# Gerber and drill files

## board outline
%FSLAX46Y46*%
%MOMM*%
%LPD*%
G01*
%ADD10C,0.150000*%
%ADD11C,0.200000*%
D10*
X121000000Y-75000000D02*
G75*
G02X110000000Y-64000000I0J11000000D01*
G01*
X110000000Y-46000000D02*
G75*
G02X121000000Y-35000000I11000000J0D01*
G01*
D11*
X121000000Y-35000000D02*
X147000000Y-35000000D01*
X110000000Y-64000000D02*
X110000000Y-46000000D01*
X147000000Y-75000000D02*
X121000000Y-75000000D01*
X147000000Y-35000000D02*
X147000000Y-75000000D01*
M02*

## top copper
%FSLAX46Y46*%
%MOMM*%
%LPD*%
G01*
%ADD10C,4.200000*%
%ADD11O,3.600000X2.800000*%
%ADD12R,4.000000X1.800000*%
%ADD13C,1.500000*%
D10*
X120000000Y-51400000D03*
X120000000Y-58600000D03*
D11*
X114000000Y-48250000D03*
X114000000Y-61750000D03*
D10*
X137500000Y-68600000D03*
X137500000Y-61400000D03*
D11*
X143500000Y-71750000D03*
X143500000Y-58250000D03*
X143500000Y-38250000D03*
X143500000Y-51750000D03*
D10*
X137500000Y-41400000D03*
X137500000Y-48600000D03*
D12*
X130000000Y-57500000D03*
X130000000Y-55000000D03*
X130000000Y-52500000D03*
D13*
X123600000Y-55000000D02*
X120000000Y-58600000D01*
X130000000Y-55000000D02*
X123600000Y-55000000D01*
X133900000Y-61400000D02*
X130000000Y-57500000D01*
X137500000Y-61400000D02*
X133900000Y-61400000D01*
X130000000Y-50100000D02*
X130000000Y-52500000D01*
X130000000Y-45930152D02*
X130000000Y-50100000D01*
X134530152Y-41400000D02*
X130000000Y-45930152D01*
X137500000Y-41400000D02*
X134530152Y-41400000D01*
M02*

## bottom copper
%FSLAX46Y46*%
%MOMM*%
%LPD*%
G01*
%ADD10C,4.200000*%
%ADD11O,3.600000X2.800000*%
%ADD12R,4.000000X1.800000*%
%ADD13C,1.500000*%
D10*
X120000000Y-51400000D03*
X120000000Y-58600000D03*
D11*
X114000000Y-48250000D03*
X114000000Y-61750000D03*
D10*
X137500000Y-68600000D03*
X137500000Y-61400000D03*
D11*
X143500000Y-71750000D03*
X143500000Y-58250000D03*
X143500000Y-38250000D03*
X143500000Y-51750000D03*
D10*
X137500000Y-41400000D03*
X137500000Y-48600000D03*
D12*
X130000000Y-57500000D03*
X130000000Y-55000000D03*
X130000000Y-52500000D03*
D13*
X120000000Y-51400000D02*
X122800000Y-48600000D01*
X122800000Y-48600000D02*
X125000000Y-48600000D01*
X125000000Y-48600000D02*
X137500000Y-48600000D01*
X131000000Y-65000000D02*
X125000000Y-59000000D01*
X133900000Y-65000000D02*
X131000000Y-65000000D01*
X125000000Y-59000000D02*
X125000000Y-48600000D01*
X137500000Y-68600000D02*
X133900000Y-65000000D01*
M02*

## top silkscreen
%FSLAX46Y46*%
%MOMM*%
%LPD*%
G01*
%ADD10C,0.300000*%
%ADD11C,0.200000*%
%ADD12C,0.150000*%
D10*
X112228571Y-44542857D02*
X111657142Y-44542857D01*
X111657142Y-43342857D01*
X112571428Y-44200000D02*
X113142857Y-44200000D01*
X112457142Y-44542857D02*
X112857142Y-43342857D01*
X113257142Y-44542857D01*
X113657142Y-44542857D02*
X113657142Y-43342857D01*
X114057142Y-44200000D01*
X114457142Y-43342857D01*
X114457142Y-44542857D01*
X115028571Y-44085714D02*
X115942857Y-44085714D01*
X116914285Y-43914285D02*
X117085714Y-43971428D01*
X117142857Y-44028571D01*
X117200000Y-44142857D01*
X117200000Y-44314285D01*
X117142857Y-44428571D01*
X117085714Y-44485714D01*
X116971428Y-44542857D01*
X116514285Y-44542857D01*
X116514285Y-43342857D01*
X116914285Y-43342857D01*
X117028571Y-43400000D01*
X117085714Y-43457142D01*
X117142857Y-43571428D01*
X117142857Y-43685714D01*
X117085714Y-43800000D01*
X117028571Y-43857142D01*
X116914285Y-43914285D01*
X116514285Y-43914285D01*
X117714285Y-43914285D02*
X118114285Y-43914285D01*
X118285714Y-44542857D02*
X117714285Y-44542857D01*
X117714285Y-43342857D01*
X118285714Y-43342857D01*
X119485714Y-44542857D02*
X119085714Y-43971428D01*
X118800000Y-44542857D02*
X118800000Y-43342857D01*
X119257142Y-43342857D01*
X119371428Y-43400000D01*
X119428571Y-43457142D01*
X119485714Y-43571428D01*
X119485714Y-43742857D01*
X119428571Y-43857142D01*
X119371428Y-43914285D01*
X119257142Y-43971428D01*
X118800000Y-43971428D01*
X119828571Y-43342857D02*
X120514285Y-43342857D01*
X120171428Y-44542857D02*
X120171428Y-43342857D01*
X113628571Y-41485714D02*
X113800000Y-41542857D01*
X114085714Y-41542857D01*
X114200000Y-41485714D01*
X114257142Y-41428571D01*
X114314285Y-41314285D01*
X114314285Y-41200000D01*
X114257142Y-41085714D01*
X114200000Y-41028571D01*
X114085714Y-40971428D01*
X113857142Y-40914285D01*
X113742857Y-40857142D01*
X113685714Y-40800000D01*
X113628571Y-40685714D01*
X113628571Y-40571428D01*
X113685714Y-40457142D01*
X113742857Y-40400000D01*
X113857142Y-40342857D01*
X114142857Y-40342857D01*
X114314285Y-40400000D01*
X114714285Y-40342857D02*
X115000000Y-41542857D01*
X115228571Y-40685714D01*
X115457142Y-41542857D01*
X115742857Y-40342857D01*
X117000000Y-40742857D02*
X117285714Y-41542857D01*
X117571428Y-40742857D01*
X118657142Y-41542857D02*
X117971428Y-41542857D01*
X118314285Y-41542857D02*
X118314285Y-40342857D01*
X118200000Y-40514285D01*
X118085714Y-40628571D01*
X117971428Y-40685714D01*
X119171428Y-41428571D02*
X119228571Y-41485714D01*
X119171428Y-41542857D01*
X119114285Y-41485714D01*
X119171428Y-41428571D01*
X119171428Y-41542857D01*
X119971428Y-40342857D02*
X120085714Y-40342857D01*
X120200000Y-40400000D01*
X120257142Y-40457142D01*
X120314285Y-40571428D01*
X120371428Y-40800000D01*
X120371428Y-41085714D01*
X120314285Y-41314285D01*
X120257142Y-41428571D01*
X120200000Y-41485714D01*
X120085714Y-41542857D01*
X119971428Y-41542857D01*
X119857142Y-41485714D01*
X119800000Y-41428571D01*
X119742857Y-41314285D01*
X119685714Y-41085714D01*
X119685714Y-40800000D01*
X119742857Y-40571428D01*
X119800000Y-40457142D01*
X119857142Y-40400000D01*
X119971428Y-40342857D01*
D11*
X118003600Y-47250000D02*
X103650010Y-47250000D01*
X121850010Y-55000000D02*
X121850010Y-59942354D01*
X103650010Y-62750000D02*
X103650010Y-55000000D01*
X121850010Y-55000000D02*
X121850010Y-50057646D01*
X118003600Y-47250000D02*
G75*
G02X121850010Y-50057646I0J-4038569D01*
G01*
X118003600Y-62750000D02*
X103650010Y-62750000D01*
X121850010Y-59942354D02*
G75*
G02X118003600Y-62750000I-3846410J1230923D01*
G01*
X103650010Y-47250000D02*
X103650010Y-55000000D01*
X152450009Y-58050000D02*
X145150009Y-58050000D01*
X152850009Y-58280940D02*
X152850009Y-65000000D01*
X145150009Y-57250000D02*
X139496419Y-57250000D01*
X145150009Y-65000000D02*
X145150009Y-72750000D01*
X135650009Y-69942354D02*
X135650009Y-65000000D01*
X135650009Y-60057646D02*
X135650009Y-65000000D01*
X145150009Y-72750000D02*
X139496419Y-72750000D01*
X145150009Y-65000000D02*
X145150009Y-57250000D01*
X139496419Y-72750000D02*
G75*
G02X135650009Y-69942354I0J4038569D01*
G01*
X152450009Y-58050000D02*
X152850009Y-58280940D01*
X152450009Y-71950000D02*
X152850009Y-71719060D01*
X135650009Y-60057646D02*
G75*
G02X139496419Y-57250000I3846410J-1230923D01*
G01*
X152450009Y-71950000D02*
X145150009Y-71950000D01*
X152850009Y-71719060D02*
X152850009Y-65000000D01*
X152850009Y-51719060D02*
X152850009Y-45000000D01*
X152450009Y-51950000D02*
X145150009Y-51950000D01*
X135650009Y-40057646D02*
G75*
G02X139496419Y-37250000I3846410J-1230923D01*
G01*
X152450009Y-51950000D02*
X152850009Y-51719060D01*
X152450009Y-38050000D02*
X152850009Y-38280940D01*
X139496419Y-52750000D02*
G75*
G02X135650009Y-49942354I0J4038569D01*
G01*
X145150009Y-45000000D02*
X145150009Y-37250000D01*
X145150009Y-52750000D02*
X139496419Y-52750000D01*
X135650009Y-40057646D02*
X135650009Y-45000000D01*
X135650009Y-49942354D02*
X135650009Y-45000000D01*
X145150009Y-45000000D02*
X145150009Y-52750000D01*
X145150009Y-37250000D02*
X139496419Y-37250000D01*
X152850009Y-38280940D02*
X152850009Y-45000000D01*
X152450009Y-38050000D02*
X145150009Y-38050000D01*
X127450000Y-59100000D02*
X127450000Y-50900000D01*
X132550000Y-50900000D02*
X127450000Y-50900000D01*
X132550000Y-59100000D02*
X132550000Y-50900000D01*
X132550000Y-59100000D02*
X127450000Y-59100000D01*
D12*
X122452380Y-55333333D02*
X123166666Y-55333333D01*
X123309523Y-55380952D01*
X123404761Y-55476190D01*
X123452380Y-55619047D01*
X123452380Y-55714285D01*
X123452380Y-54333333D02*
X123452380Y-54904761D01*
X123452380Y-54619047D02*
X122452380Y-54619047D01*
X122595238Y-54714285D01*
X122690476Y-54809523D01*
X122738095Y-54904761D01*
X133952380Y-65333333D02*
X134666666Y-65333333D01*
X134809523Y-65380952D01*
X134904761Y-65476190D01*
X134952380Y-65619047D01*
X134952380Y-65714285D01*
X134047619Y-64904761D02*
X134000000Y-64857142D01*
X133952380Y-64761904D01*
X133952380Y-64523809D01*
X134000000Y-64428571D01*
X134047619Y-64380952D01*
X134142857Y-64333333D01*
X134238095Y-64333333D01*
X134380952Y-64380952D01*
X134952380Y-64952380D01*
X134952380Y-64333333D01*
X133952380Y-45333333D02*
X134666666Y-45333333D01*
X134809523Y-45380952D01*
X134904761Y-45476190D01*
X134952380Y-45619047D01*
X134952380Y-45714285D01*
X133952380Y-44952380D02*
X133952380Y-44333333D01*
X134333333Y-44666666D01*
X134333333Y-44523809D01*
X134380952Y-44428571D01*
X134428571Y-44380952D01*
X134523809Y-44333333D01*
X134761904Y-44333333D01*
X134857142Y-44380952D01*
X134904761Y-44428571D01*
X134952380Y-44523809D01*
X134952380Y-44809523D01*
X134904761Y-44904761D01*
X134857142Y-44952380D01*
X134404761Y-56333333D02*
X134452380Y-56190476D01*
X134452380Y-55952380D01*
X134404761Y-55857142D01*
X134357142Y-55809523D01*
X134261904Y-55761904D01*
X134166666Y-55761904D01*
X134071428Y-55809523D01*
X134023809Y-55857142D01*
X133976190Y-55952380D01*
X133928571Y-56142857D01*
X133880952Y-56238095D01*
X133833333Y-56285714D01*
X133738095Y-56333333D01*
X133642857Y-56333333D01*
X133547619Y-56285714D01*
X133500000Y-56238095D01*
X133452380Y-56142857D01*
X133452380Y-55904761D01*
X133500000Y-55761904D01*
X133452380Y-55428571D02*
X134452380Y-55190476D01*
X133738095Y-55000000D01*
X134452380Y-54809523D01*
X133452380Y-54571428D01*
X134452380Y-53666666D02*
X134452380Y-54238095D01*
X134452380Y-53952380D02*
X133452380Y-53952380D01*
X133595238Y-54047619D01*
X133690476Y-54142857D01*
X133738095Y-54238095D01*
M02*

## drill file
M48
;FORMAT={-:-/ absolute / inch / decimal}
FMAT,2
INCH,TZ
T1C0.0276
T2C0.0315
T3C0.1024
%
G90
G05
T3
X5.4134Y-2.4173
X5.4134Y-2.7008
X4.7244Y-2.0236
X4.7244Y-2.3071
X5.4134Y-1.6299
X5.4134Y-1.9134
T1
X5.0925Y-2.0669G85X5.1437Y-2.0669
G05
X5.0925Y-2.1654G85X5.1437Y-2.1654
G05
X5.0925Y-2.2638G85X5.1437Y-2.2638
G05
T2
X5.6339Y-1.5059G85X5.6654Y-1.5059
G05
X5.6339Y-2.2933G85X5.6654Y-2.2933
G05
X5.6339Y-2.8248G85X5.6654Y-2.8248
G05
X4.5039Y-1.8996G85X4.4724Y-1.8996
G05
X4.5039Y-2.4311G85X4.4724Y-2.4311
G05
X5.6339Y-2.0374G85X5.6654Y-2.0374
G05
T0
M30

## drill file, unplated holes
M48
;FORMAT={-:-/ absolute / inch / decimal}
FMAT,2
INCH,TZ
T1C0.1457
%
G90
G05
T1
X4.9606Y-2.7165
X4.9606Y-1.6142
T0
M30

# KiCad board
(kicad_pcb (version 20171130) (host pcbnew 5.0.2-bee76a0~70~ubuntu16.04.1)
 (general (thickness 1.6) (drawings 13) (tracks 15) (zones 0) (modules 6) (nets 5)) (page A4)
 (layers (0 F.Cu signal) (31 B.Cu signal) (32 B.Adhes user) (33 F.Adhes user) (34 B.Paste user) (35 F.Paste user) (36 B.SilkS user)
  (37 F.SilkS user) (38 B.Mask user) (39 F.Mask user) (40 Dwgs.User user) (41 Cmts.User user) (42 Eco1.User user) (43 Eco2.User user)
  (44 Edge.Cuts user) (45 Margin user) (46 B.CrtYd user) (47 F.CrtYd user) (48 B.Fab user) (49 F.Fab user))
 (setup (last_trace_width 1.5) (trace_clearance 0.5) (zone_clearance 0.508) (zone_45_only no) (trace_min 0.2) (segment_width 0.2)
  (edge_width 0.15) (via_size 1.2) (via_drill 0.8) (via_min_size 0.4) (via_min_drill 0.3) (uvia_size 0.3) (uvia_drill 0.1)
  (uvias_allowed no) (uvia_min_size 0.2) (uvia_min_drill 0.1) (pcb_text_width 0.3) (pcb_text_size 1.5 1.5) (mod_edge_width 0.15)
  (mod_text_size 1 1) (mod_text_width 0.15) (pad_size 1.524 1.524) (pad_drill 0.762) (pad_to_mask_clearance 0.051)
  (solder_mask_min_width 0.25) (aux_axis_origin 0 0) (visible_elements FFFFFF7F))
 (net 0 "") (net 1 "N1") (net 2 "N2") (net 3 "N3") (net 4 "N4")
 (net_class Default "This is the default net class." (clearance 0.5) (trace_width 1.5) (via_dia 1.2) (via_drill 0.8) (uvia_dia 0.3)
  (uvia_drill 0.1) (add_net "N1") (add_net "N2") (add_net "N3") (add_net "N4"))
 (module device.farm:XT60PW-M (layer F.Cu) (at 120 55 270)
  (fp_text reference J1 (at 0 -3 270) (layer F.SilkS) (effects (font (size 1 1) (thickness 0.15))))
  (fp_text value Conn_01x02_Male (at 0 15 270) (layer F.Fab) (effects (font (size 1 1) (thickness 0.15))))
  (fp_line (start -7.75 1.9964) (end -7.75 16.34999) (layer F.SilkS) (width 0.2))
  (fp_line (start 0 -1.85001) (end 4.942354 -1.85001) (layer F.SilkS) (width 0.2))
  (fp_line (start 7.75 16.34999) (end 0 16.34999) (layer F.SilkS) (width 0.2))
  (fp_line (start 0 -1.85001) (end -4.942354 -1.85001) (layer F.SilkS) (width 0.2))
  (fp_arc (start -3.711431 1.9964) (end -4.942354 -1.85001) (angle -72.25435427) (layer F.SilkS) (width 0.2))
  (fp_line (start 7.75 1.9964) (end 7.75 16.34999) (layer F.SilkS) (width 0.2))
  (fp_arc (start 3.711431 1.9964) (end 7.75 1.9964) (angle -72.25435427) (layer F.SilkS) (width 0.2))
  (fp_line (start -7.75 16.34999) (end 0 16.34999) (layer F.SilkS) (width 0.2))
  (pad 1 thru_hole circle (at -3.6 0 270) (size 4.2 4.2) (drill 2.6) (layers *.Cu *.Mask) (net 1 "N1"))
  (pad 2 thru_hole circle (at 3.6 0 270) (size 4.2 4.2) (drill 2.6) (layers *.Cu *.Mask) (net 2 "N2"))
  (pad "" thru_hole oval (at -6.75 6 270) (size 2.8 3.6) (drill oval 0.8 1.6) (layers *.Cu *.Mask))
  (pad "" thru_hole oval (at 6.75 6 270) (size 2.8 3.6) (drill oval 0.8 1.6) (layers *.Cu *.Mask)))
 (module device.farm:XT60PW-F (layer F.Cu) (at 137.5 65 90)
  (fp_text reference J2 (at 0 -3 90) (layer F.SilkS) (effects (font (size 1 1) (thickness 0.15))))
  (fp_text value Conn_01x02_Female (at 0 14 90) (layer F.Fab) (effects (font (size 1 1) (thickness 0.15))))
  (fp_line (start 6.95 14.950009) (end 6.95 7.650009) (layer F.SilkS) (width 0.2))
  (fp_line (start 6.71906 15.350009) (end 0 15.350009) (layer F.SilkS) (width 0.2))
  (fp_line (start 7.75 7.650009) (end 7.75 1.996419) (layer F.SilkS) (width 0.2))
  (fp_line (start 0 7.650009) (end -7.75 7.650009) (layer F.SilkS) (width 0.2))
  (fp_line (start -4.942354 -1.849991) (end 0 -1.849991) (layer F.SilkS) (width 0.2))
  (fp_line (start 4.942354 -1.849991) (end 0 -1.849991) (layer F.SilkS) (width 0.2))
  (fp_line (start -7.75 7.650009) (end -7.75 1.996419) (layer F.SilkS) (width 0.2))
  (fp_line (start 0 7.650009) (end 7.75 7.650009) (layer F.SilkS) (width 0.2))
  (fp_arc (start -3.711431 1.996419) (end -4.942354 -1.849991) (angle -72.25435427) (layer F.SilkS) (width 0.2))
  (fp_line (start 6.95 14.950009) (end 6.71906 15.350009) (layer F.SilkS) (width 0.2))
  (fp_line (start -6.95 14.950009) (end -6.71906 15.350009) (layer F.SilkS) (width 0.2))
  (fp_arc (start 3.711431 1.996419) (end 7.75 1.996419) (angle -72.25435427) (layer F.SilkS) (width 0.2))
  (fp_line (start -6.95 14.950009) (end -6.95 7.650009) (layer F.SilkS) (width 0.2))
  (fp_line (start -6.71906 15.350009) (end 0 15.350009) (layer F.SilkS) (width 0.2))
  (pad 1 thru_hole circle (at -3.6 0 90) (size 4.2 4.2) (drill 2.6) (layers *.Cu *.Mask) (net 1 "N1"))
  (pad 2 thru_hole circle (at 3.6 0 90) (size 4.2 4.2) (drill 2.6) (layers *.Cu *.Mask) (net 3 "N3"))
  (pad "" thru_hole oval (at -6.75 6 90) (size 2.8 3.6) (drill oval 0.8 1.6) (layers *.Cu *.Mask))
  (pad "" thru_hole oval (at 6.75 6 90) (size 2.8 3.6) (drill oval 0.8 1.6) (layers *.Cu *.Mask)))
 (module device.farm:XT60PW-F (layer F.Cu) (at 137.5 45 90)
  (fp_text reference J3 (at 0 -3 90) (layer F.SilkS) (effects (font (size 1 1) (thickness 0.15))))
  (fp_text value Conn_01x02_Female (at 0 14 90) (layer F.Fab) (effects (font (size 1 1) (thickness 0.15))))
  (fp_line (start -6.71906 15.350009) (end 0 15.350009) (layer F.SilkS) (width 0.2))
  (fp_line (start -6.95 14.950009) (end -6.95 7.650009) (layer F.SilkS) (width 0.2))
  (fp_arc (start 3.711431 1.996419) (end 7.75 1.996419) (angle -72.25435427) (layer F.SilkS) (width 0.2))
  (fp_line (start -6.95 14.950009) (end -6.71906 15.350009) (layer F.SilkS) (width 0.2))
  (fp_line (start 6.95 14.950009) (end 6.71906 15.350009) (layer F.SilkS) (width 0.2))
  (fp_arc (start -3.711431 1.996419) (end -4.942354 -1.849991) (angle -72.25435427) (layer F.SilkS) (width 0.2))
  (fp_line (start 0 7.650009) (end 7.75 7.650009) (layer F.SilkS) (width 0.2))
  (fp_line (start -7.75 7.650009) (end -7.75 1.996419) (layer F.SilkS) (width 0.2))
  (fp_line (start 4.942354 -1.849991) (end 0 -1.849991) (layer F.SilkS) (width 0.2))
  (fp_line (start -4.942354 -1.849991) (end 0 -1.849991) (layer F.SilkS) (width 0.2))
  (fp_line (start 0 7.650009) (end -7.75 7.650009) (layer F.SilkS) (width 0.2))
  (fp_line (start 7.75 7.650009) (end 7.75 1.996419) (layer F.SilkS) (width 0.2))
  (fp_line (start 6.71906 15.350009) (end 0 15.350009) (layer F.SilkS) (width 0.2))
  (fp_line (start 6.95 14.950009) (end 6.95 7.650009) (layer F.SilkS) (width 0.2))
  (pad "" thru_hole oval (at 6.75 6 90) (size 2.8 3.6) (drill oval 0.8 1.6) (layers *.Cu *.Mask))
  (pad "" thru_hole oval (at -6.75 6 90) (size 2.8 3.6) (drill oval 0.8 1.6) (layers *.Cu *.Mask))
  (pad 2 thru_hole circle (at 3.6 0 90) (size 4.2 4.2) (drill 2.6) (layers *.Cu *.Mask) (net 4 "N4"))
  (pad 1 thru_hole circle (at -3.6 0 90) (size 4.2 4.2) (drill 2.6) (layers *.Cu *.Mask) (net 1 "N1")))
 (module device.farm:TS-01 (layer F.Cu) (at 130 55 90)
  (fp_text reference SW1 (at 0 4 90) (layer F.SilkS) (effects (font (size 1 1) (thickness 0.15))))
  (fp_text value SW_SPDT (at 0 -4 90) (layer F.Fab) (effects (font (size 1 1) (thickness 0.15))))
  (fp_line (start -4.1 -2.55) (end 4.1 -2.55) (layer F.SilkS) (width 0.2))
  (fp_line (start 4.1 2.55) (end 4.1 -2.55) (layer F.SilkS) (width 0.2))
  (fp_line (start -4.1 2.55) (end 4.1 2.55) (layer F.SilkS) (width 0.2))
  (fp_line (start -4.1 2.55) (end -4.1 -2.55) (layer F.SilkS) (width 0.2))
  (pad 1 thru_hole rect (at -2.5 0 90) (size 1.8 4) (drill oval 0.7 2) (layers *.Cu *.Mask) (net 3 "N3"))
  (pad 2 thru_hole rect (at 0 0 90) (size 1.8 4) (drill oval 0.7 2) (layers *.Cu *.Mask) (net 2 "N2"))
  (pad 3 thru_hole rect (at 2.5 0 90) (size 1.8 4) (drill oval 0.7 2) (layers *.Cu *.Mask) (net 4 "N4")))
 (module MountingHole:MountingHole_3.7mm (layer F.Cu) (at 126 41)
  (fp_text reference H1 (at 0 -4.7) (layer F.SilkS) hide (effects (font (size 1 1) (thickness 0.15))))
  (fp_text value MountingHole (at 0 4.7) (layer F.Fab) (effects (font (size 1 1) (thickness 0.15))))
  (pad 1 np_thru_hole circle (at 0 0) (size 3.7 3.7) (drill 3.7) (layers *.Cu *.Mask)))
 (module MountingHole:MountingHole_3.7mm (layer F.Cu) (at 126 69)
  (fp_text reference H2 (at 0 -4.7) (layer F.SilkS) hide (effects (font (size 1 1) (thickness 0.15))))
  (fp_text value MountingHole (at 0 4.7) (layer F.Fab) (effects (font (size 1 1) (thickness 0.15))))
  (pad 1 np_thru_hole circle (at 0 0) (size 3.7 3.7) (drill 3.7) (layers *.Cu *.Mask)))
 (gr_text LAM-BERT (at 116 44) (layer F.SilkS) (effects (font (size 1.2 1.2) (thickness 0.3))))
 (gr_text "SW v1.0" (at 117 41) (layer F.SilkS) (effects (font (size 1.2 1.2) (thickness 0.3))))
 (gr_arc (start 121 64) (end 110 64) (angle -90) (layer Edge.Cuts) (width 0.15))
 (gr_arc (start 121 46) (end 121 35) (angle -90) (layer Edge.Cuts) (width 0.15))
 (gr_line (start 121 35) (end 147 35) (layer Edge.Cuts) (width 0.2))
 (gr_line (start 110 64) (end 110 46) (layer Edge.Cuts) (width 0.2))
 (gr_line (start 147 75) (end 121 75) (layer Edge.Cuts) (width 0.2))
 (gr_line (start 147 35) (end 147 75) (layer Edge.Cuts) (width 0.2))
 (segment (start 120 51.4) (end 122.8 48.6) (width 1.5) (layer B.Cu) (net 1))
 (segment (start 122.8 48.6) (end 125 48.6) (width 1.5) (layer B.Cu) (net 1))
 (segment (start 125 48.6) (end 137.5 48.6) (width 1.5) (layer B.Cu) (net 1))
 (segment (start 131 65) (end 125 59) (width 1.5) (layer B.Cu) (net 1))
 (segment (start 133.9 65) (end 131 65) (width 1.5) (layer B.Cu) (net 1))
 (segment (start 125 59) (end 125 48.6) (width 1.5) (layer B.Cu) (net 1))
 (segment (start 137.5 68.6) (end 133.9 65) (width 1.5) (layer B.Cu) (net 1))
 (segment (start 123.6 55) (end 120 58.6) (width 1.5) (layer F.Cu) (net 2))
 (segment (start 130 55) (end 123.6 55) (width 1.5) (layer F.Cu) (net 2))
 (segment (start 133.9 61.4) (end 130 57.5) (width 1.5) (layer F.Cu) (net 3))
 (segment (start 137.5 61.4) (end 133.9 61.4) (width 1.5) (layer F.Cu) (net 3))
 (segment (start 130 50.1) (end 130 52.5) (width 1.5) (layer F.Cu) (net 4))
 (segment (start 130 45.930152) (end 130 50.1) (width 1.5) (layer F.Cu) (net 4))
 (segment (start 134.530152 41.4) (end 130 45.930152) (width 1.5) (layer F.Cu) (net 4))
 (segment (start 137.5 41.4) (end 134.530152 41.4) (width 1.5) (layer F.Cu) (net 4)))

